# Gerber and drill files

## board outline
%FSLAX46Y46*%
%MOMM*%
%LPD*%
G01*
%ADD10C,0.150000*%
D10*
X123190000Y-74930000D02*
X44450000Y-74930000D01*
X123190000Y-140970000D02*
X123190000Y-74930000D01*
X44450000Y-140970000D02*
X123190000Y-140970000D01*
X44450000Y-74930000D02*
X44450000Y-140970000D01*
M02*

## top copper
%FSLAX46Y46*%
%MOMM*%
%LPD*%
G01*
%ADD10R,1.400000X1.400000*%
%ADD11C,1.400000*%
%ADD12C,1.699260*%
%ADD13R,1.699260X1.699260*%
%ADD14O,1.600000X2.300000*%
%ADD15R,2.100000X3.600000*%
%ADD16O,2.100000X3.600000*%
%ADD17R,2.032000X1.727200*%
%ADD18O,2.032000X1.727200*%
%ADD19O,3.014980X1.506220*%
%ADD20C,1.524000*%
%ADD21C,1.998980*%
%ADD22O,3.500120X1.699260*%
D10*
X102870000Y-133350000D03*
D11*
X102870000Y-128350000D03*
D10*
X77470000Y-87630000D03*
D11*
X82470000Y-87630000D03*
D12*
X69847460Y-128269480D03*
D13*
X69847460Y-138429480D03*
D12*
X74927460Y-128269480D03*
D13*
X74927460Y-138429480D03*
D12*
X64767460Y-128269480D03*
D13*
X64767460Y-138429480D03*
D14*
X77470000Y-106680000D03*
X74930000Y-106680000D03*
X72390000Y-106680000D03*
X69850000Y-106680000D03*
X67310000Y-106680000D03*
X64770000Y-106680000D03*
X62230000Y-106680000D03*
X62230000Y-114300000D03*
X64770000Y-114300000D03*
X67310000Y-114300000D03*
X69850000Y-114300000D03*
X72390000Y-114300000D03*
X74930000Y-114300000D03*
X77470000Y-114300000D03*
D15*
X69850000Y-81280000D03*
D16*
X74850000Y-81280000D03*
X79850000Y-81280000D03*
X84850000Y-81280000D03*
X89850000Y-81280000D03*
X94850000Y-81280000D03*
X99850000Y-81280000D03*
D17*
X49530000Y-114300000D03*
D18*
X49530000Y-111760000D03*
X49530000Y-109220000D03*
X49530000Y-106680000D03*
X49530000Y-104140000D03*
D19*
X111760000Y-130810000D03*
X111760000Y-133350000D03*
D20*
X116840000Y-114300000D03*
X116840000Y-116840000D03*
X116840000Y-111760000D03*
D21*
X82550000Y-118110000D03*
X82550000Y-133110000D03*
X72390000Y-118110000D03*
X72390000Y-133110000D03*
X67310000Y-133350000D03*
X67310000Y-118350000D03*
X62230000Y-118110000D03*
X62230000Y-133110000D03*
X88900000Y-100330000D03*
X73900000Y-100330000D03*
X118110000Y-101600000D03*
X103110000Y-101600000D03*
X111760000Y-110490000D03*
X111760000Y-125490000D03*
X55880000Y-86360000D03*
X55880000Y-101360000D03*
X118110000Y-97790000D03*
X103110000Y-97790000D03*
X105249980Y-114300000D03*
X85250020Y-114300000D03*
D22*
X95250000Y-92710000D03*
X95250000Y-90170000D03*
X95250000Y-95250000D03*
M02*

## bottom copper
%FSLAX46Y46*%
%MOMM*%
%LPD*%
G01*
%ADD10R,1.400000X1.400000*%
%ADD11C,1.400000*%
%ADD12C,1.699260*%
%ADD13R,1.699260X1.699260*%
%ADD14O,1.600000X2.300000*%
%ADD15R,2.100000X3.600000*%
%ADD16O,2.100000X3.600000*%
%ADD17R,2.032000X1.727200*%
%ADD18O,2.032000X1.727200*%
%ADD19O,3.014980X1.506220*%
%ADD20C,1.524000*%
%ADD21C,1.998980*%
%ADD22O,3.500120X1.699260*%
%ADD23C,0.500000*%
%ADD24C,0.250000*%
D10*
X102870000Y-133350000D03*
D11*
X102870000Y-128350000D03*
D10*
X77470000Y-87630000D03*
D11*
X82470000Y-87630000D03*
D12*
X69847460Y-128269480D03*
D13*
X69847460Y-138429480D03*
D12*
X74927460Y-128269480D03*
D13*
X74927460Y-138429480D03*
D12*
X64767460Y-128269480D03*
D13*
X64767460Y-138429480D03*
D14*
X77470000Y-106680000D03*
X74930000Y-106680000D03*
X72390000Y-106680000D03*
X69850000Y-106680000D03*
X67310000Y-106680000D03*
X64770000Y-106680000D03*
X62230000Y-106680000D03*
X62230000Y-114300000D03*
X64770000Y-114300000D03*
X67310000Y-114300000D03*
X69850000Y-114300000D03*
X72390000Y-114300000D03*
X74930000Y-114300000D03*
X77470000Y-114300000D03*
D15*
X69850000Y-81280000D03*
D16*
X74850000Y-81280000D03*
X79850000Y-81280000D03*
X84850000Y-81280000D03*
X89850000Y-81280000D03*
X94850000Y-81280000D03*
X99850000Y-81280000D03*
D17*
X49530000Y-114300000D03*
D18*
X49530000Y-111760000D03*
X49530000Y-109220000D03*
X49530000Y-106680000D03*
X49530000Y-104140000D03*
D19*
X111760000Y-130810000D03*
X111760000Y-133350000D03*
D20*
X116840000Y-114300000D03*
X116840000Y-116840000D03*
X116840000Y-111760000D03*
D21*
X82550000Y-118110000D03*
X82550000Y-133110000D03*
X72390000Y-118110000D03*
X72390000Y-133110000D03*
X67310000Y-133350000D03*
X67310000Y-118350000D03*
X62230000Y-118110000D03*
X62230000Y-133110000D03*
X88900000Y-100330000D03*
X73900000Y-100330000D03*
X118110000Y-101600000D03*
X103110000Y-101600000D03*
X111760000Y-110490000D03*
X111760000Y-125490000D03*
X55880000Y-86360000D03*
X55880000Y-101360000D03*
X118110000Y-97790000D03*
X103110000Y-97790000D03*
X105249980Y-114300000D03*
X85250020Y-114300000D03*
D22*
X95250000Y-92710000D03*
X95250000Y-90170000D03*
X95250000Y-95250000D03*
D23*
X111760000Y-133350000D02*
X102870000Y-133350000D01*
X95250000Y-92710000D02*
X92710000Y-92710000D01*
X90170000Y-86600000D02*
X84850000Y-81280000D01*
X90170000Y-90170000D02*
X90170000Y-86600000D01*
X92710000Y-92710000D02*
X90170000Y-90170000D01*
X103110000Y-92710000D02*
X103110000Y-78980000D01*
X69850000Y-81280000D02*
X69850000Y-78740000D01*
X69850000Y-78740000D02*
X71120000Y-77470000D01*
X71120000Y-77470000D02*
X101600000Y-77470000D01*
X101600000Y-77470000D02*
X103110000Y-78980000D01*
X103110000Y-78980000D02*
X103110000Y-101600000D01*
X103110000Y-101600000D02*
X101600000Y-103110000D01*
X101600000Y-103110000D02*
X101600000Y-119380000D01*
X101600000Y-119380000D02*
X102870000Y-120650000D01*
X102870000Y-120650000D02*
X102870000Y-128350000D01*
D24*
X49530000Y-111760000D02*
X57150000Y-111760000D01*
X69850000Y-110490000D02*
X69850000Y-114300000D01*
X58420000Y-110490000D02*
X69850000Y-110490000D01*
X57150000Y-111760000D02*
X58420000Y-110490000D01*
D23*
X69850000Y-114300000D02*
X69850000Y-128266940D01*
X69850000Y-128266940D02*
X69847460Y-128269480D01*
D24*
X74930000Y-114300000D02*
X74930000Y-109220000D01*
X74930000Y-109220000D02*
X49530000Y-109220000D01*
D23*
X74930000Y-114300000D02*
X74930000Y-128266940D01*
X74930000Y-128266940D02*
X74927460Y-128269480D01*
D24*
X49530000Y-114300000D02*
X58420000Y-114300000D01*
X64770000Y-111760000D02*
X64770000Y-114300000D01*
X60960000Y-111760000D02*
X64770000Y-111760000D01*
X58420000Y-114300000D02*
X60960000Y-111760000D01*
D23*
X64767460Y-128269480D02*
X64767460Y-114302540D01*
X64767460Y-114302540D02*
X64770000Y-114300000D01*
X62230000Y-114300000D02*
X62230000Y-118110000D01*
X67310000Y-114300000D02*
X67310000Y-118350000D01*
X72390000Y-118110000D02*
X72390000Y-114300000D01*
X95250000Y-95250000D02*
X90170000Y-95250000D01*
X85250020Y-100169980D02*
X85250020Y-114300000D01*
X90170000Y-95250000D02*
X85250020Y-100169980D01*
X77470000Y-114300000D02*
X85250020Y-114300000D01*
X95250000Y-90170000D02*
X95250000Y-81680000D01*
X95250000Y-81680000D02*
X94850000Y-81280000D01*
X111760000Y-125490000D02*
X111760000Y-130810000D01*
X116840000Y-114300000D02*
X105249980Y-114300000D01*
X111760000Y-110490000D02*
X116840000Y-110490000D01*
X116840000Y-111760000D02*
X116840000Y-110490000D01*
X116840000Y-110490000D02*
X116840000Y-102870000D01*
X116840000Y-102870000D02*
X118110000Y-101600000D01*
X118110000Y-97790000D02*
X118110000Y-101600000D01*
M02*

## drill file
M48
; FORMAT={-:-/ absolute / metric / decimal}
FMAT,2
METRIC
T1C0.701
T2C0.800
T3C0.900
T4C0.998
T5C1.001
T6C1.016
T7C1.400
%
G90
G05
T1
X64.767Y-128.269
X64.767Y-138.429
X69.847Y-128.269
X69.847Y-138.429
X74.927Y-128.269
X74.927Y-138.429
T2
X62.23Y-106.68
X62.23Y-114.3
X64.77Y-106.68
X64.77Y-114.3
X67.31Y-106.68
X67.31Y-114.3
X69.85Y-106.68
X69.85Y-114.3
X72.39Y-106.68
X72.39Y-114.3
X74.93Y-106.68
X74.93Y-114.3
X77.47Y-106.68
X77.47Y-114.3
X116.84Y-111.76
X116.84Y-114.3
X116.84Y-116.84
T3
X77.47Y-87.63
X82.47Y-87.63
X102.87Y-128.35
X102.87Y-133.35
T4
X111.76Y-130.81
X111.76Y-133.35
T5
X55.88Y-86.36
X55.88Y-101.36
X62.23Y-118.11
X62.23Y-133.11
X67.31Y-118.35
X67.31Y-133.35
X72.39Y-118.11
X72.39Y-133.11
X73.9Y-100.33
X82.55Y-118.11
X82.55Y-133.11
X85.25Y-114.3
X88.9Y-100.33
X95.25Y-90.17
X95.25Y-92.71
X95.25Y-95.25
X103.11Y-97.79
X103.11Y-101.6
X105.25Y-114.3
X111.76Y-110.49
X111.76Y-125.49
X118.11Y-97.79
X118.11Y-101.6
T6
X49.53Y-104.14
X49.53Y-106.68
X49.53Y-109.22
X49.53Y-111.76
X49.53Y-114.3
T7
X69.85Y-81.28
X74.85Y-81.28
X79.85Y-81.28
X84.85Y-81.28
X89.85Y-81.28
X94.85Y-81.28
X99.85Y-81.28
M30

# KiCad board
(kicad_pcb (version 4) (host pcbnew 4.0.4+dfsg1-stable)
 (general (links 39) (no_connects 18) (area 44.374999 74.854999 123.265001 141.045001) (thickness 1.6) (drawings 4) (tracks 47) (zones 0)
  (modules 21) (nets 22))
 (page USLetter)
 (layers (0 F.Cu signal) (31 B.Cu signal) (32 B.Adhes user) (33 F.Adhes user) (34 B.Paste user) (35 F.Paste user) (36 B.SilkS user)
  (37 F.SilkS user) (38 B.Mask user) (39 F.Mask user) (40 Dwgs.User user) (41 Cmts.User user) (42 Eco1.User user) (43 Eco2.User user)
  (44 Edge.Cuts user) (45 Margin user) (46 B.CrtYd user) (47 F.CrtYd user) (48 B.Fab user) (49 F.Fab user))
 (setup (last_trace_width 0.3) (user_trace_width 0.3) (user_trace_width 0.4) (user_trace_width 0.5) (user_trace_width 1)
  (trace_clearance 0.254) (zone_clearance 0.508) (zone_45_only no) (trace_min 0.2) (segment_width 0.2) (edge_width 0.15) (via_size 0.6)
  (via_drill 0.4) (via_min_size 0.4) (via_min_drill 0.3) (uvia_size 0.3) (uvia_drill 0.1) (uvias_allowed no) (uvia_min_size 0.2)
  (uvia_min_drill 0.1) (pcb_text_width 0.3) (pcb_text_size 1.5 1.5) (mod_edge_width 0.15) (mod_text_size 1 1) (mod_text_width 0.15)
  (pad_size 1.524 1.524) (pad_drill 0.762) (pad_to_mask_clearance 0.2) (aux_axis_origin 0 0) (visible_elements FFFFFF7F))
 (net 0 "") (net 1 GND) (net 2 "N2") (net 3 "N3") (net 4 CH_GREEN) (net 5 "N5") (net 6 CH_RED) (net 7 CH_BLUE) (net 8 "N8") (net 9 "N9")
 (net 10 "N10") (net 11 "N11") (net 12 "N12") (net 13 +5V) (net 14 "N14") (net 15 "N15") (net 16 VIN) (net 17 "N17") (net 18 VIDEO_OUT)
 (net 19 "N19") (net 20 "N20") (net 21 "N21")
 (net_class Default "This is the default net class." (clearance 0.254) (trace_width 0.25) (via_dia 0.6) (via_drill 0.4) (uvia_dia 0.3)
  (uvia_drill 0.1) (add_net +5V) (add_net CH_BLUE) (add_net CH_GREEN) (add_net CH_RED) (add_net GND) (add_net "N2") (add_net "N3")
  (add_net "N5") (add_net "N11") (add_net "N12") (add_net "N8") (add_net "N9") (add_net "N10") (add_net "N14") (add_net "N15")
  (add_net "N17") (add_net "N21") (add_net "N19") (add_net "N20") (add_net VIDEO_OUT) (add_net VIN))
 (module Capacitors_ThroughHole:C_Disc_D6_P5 (layer F.Cu) (at 102.87 133.35 90)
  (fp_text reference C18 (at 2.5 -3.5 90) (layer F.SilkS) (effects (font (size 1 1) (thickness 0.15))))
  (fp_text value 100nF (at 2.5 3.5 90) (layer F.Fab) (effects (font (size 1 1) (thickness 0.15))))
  (pad 1 thru_hole rect (at 0 0 90) (size 1.4 1.4) (drill 0.9) (layers *.Cu *.Mask F.SilkS) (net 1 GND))
  (pad 2 thru_hole circle (at 5 0 90) (size 1.4 1.4) (drill 0.9) (layers *.Cu *.Mask F.SilkS) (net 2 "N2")))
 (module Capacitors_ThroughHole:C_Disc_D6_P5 (layer F.Cu) (at 77.47 87.63)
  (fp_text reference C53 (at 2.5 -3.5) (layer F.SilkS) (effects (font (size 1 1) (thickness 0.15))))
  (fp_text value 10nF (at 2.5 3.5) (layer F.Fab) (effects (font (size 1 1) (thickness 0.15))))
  (pad 1 thru_hole rect (at 0 0) (size 1.4 1.4) (drill 0.9) (layers *.Cu *.Mask F.SilkS) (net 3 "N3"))
  (pad 2 thru_hole circle (at 5 0) (size 1.4 1.4) (drill 0.9) (layers *.Cu *.Mask F.SilkS) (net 1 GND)))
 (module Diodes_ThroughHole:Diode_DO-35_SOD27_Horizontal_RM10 (layer F.Cu) (at 69.85 138.43 90)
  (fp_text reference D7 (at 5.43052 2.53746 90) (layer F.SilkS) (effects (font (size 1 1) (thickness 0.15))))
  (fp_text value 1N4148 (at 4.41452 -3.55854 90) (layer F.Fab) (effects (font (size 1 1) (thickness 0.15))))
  (pad 2 thru_hole circle (at 10.16052 -0.00254 270) (size 1.69926 1.69926) (drill 0.70104) (layers *.Cu *.Mask F.SilkS) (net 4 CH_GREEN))
  (pad 1 thru_hole rect (at 0.00052 -0.00254 270) (size 1.69926 1.69926) (drill 0.70104) (layers *.Cu *.Mask F.SilkS) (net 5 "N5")))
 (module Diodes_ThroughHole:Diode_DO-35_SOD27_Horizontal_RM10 (layer F.Cu) (at 74.93 138.43 90)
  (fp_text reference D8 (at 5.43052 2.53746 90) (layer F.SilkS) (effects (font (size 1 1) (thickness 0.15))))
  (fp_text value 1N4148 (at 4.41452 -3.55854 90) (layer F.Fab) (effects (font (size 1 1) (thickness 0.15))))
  (pad 2 thru_hole circle (at 10.16052 -0.00254 270) (size 1.69926 1.69926) (drill 0.70104) (layers *.Cu *.Mask F.SilkS) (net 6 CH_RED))
  (pad 1 thru_hole rect (at 0.00052 -0.00254 270) (size 1.69926 1.69926) (drill 0.70104) (layers *.Cu *.Mask F.SilkS) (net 5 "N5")))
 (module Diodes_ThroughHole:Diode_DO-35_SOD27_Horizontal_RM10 (layer F.Cu) (at 64.77 138.43 90)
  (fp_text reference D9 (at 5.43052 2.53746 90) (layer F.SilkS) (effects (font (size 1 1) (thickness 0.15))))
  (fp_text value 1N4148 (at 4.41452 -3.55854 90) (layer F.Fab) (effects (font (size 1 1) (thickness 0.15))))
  (pad 2 thru_hole circle (at 10.16052 -0.00254 270) (size 1.69926 1.69926) (drill 0.70104) (layers *.Cu *.Mask F.SilkS) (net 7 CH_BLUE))
  (pad 1 thru_hole rect (at 0.00052 -0.00254 270) (size 1.69926 1.69926) (drill 0.70104) (layers *.Cu *.Mask F.SilkS) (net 5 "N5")))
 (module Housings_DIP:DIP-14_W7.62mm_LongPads (layer F.Cu) (at 77.47 106.68 270)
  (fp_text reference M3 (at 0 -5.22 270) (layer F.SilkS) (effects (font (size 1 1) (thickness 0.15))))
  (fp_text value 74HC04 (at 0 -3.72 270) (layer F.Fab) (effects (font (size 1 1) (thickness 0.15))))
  (pad 1 thru_hole oval (at 0 0 270) (size 2.3 1.6) (drill 0.8) (layers *.Cu *.Mask F.SilkS))
  (pad 2 thru_hole oval (at 0 2.54 270) (size 2.3 1.6) (drill 0.8) (layers *.Cu *.Mask F.SilkS))
  (pad 3 thru_hole oval (at 0 5.08 270) (size 2.3 1.6) (drill 0.8) (layers *.Cu *.Mask F.SilkS))
  (pad 4 thru_hole oval (at 0 7.62 270) (size 2.3 1.6) (drill 0.8) (layers *.Cu *.Mask F.SilkS))
  (pad 5 thru_hole oval (at 0 10.16 270) (size 2.3 1.6) (drill 0.8) (layers *.Cu *.Mask F.SilkS) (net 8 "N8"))
  (pad 6 thru_hole oval (at 0 12.7 270) (size 2.3 1.6) (drill 0.8) (layers *.Cu *.Mask F.SilkS) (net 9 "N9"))
  (pad 7 thru_hole oval (at 0 15.24 270) (size 2.3 1.6) (drill 0.8) (layers *.Cu *.Mask F.SilkS) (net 1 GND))
  (pad 8 thru_hole oval (at 7.62 15.24 270) (size 2.3 1.6) (drill 0.8) (layers *.Cu *.Mask F.SilkS) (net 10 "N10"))
  (pad 9 thru_hole oval (at 7.62 12.7 270) (size 2.3 1.6) (drill 0.8) (layers *.Cu *.Mask F.SilkS) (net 7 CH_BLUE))
  (pad 10 thru_hole oval (at 7.62 10.16 270) (size 2.3 1.6) (drill 0.8) (layers *.Cu *.Mask F.SilkS) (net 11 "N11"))
  (pad 11 thru_hole oval (at 7.62 7.62 270) (size 2.3 1.6) (drill 0.8) (layers *.Cu *.Mask F.SilkS) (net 4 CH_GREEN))
  (pad 12 thru_hole oval (at 7.62 5.08 270) (size 2.3 1.6) (drill 0.8) (layers *.Cu *.Mask F.SilkS) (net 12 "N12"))
  (pad 13 thru_hole oval (at 7.62 2.54 270) (size 2.3 1.6) (drill 0.8) (layers *.Cu *.Mask F.SilkS) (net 6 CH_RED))
  (pad 14 thru_hole oval (at 7.62 0 270) (size 2.3 1.6) (drill 0.8) (layers *.Cu *.Mask F.SilkS) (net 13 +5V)))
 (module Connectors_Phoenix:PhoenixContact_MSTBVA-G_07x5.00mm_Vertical (layer F.Cu) (at 69.85 81.28)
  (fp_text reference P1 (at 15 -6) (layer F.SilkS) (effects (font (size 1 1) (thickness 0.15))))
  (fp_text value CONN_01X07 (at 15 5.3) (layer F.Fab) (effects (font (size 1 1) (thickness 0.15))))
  (pad 1 thru_hole rect (at 0 0) (size 2.1 3.6) (drill 1.4) (layers *.Cu *.Mask) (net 2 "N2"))
  (pad 2 thru_hole oval (at 5 0) (size 2.1 3.6) (drill 1.4) (layers *.Cu *.Mask) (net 3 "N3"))
  (pad 3 thru_hole oval (at 10 0) (size 2.1 3.6) (drill 1.4) (layers *.Cu *.Mask) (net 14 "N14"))
  (pad 4 thru_hole oval (at 15 0) (size 2.1 3.6) (drill 1.4) (layers *.Cu *.Mask) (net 1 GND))
  (pad 5 thru_hole oval (at 20 0) (size 2.1 3.6) (drill 1.4) (layers *.Cu *.Mask) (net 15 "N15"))
  (pad 6 thru_hole oval (at 25 0) (size 2.1 3.6) (drill 1.4) (layers *.Cu *.Mask) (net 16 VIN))
  (pad 7 thru_hole oval (at 30 0) (size 2.1 3.6) (drill 1.4) (layers *.Cu *.Mask) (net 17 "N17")))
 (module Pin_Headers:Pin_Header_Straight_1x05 (layer B.Cu) (at 49.53 114.3)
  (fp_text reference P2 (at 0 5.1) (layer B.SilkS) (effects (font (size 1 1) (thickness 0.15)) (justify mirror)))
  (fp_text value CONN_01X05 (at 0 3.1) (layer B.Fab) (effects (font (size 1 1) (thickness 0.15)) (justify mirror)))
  (pad 1 thru_hole rect (at 0 0) (size 2.032 1.7272) (drill 1.016) (layers *.Cu *.Mask B.SilkS) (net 7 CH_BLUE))
  (pad 2 thru_hole oval (at 0 -2.54) (size 2.032 1.7272) (drill 1.016) (layers *.Cu *.Mask B.SilkS) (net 4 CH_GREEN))
  (pad 3 thru_hole oval (at 0 -5.08) (size 2.032 1.7272) (drill 1.016) (layers *.Cu *.Mask B.SilkS) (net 6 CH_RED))
  (pad 4 thru_hole oval (at 0 -7.62) (size 2.032 1.7272) (drill 1.016) (layers *.Cu *.Mask B.SilkS) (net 13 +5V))
  (pad 5 thru_hole oval (at 0 -10.16) (size 2.032 1.7272) (drill 1.016) (layers *.Cu *.Mask B.SilkS) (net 1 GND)))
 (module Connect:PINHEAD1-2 (layer F.Cu) (at 111.76 132.08 270)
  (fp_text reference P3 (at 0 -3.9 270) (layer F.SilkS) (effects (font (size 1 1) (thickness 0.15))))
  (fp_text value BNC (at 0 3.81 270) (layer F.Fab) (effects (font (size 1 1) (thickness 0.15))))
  (pad 1 thru_hole oval (at -1.27 0 270) (size 1.50622 3.01498) (drill 0.99822) (layers *.Cu *.Mask) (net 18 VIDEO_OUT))
  (pad 2 thru_hole oval (at 1.27 0 270) (size 1.50622 3.01498) (drill 0.99822) (layers *.Cu *.Mask) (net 1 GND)))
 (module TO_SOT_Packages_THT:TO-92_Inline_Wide (layer F.Cu) (at 116.84 111.76 270)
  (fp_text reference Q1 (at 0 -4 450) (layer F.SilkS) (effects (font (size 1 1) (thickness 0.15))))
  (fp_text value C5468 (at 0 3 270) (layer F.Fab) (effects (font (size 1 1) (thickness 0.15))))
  (pad 2 thru_hole circle (at 2.54 0) (size 1.524 1.524) (drill 0.8) (layers *.Cu *.Mask F.SilkS) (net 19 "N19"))
  (pad 3 thru_hole circle (at 5.08 0) (size 1.524 1.524) (drill 0.8) (layers *.Cu *.Mask F.SilkS) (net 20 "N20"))
  (pad 1 thru_hole circle (at 0 0) (size 1.524 1.524) (drill 0.8) (layers *.Cu *.Mask F.SilkS) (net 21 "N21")))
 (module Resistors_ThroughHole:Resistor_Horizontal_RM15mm (layer F.Cu) (at 82.55 118.11 270)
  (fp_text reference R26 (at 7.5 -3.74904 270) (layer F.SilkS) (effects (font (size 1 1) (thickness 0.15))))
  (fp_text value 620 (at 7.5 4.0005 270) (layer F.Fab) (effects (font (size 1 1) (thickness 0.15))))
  (pad 1 thru_hole circle (at 0 0 270) (size 1.99898 1.99898) (drill 1.00076) (layers *.Cu *.SilkS *.Mask) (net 9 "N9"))
  (pad 2 thru_hole circle (at 15 0 270) (size 1.99898 1.99898) (drill 1.00076) (layers *.Cu *.SilkS *.Mask) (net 20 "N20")))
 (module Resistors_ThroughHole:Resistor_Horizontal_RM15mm (layer F.Cu) (at 72.39 118.11 270)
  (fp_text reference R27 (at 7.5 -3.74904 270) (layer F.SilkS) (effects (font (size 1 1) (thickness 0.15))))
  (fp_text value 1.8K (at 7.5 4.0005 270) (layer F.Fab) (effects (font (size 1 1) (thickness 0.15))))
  (pad 1 thru_hole circle (at 0 0 270) (size 1.99898 1.99898) (drill 1.00076) (layers *.Cu *.SilkS *.Mask) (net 12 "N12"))
  (pad 2 thru_hole circle (at 15 0 270) (size 1.99898 1.99898) (drill 1.00076) (layers *.Cu *.SilkS *.Mask) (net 20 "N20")))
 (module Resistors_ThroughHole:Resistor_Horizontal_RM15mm (layer F.Cu) (at 67.31 133.35 90)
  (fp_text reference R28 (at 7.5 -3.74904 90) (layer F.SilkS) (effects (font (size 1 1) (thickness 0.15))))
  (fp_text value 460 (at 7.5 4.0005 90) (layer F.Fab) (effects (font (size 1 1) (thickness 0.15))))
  (pad 1 thru_hole circle (at 0 0 90) (size 1.99898 1.99898) (drill 1.00076) (layers *.Cu *.SilkS *.Mask) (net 20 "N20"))
  (pad 2 thru_hole circle (at 15 0 90) (size 1.99898 1.99898) (drill 1.00076) (layers *.Cu *.SilkS *.Mask) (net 11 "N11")))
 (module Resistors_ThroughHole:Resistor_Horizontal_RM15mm (layer F.Cu) (at 62.23 118.11 270)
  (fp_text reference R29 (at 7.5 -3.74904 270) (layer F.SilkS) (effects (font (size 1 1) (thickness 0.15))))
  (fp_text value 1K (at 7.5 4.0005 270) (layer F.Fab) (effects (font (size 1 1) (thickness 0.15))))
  (pad 1 thru_hole circle (at 0 0 270) (size 1.99898 1.99898) (drill 1.00076) (layers *.Cu *.SilkS *.Mask) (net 10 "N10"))
  (pad 2 thru_hole circle (at 15 0 270) (size 1.99898 1.99898) (drill 1.00076) (layers *.Cu *.SilkS *.Mask) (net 20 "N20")))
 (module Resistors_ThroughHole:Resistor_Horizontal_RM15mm (layer F.Cu) (at 88.9 100.33 180)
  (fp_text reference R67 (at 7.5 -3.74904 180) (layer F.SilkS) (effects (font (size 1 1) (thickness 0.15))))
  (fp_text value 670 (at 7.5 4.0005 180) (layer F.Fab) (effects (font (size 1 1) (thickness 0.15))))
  (pad 1 thru_hole circle (at 0 0 180) (size 1.99898 1.99898) (drill 1.00076) (layers *.Cu *.SilkS *.Mask) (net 5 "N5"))
  (pad 2 thru_hole circle (at 15 0 180) (size 1.99898 1.99898) (drill 1.00076) (layers *.Cu *.SilkS *.Mask) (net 8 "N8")))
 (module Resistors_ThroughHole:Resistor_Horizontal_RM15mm (layer F.Cu) (at 118.11 101.6 180)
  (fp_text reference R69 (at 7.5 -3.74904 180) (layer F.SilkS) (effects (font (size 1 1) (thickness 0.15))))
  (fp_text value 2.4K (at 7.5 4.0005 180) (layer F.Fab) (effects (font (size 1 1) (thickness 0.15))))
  (pad 1 thru_hole circle (at 0 0 180) (size 1.99898 1.99898) (drill 1.00076) (layers *.Cu *.SilkS *.Mask) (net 21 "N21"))
  (pad 2 thru_hole circle (at 15 0 180) (size 1.99898 1.99898) (drill 1.00076) (layers *.Cu *.SilkS *.Mask) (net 2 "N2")))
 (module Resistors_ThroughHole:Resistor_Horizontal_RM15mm (layer F.Cu) (at 111.76 110.49 270)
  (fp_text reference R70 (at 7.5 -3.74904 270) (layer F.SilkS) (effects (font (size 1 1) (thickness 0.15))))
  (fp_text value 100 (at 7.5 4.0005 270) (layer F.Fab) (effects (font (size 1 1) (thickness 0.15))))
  (pad 1 thru_hole circle (at 0 0 270) (size 1.99898 1.99898) (drill 1.00076) (layers *.Cu *.SilkS *.Mask) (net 21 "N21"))
  (pad 2 thru_hole circle (at 15 0 270) (size 1.99898 1.99898) (drill 1.00076) (layers *.Cu *.SilkS *.Mask) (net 18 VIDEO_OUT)))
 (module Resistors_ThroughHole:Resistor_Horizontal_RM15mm (layer F.Cu) (at 55.88 86.36 270)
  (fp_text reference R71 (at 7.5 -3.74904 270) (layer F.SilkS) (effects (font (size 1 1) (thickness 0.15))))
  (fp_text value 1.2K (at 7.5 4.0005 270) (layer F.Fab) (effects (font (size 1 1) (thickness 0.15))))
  (pad 1 thru_hole circle (at 0 0 270) (size 1.99898 1.99898) (drill 1.00076) (layers *.Cu *.SilkS *.Mask) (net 3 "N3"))
  (pad 2 thru_hole circle (at 15 0 270) (size 1.99898 1.99898) (drill 1.00076) (layers *.Cu *.SilkS *.Mask) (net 20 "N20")))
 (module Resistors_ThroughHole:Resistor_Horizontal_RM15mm (layer F.Cu) (at 118.11 97.79 180)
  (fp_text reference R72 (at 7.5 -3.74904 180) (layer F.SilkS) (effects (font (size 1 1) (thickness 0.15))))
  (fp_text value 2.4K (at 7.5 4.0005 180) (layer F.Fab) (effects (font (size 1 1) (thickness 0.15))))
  (pad 1 thru_hole circle (at 0 0 180) (size 1.99898 1.99898) (drill 1.00076) (layers *.Cu *.SilkS *.Mask) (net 21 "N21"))
  (pad 2 thru_hole circle (at 15 0 180) (size 1.99898 1.99898) (drill 1.00076) (layers *.Cu *.SilkS *.Mask) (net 2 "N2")))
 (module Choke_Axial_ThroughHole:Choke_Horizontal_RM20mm (layer F.Cu) (at 95.25 114.3 180)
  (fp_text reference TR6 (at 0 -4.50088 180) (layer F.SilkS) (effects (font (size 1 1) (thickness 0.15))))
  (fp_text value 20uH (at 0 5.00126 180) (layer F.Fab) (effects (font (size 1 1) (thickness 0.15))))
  (pad 1 thru_hole circle (at -9.99998 0 180) (size 1.99898 1.99898) (drill 1.00076) (layers *.Cu *.Mask F.SilkS) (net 19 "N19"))
  (pad 2 thru_hole circle (at 9.99998 0 180) (size 1.99898 1.99898) (drill 1.00076) (layers *.Cu *.Mask F.SilkS) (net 13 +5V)))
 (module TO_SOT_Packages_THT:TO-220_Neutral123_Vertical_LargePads (layer F.Cu) (at 95.25 92.71 270)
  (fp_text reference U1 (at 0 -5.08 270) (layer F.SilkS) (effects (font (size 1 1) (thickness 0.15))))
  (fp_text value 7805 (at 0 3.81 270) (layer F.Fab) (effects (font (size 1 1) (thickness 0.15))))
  (pad 2 thru_hole oval (at 0 0) (size 3.50012 1.69926) (drill 1.00076) (layers *.Cu *.Mask F.SilkS) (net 1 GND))
  (pad 1 thru_hole oval (at -2.54 0) (size 3.50012 1.69926) (drill 1.00076) (layers *.Cu *.Mask F.SilkS) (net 16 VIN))
  (pad 3 thru_hole oval (at 2.54 0) (size 3.50012 1.69926) (drill 1.00076) (layers *.Cu *.Mask F.SilkS) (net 13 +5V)))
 (gr_line (start 123.19 74.93) (end 44.45 74.93) (angle 90) (layer Edge.Cuts) (width 0.15))
 (gr_line (start 123.19 140.97) (end 123.19 74.93) (angle 90) (layer Edge.Cuts) (width 0.15))
 (gr_line (start 44.45 140.97) (end 123.19 140.97) (angle 90) (layer Edge.Cuts) (width 0.15))
 (gr_line (start 44.45 74.93) (end 44.45 140.97) (angle 90) (layer Edge.Cuts) (width 0.15))
 (segment (start 111.76 133.35) (end 102.87 133.35) (width 0.5) (layer B.Cu) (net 1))
 (segment (start 95.25 92.71) (end 92.71 92.71) (width 0.5) (layer B.Cu) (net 1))
 (segment (start 90.17 86.6) (end 84.85 81.28) (width 0.5) (layer B.Cu) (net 1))
 (segment (start 90.17 90.17) (end 90.17 86.6) (width 0.5) (layer B.Cu) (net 1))
 (segment (start 92.71 92.71) (end 90.17 90.17) (width 0.5) (layer B.Cu) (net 1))
 (segment (start 103.11 92.71) (end 103.11 78.98) (width 0.5) (layer B.Cu) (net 2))
 (segment (start 69.85 81.28) (end 69.85 78.74) (width 0.5) (layer B.Cu) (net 2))
 (segment (start 69.85 78.74) (end 71.12 77.47) (width 0.5) (layer B.Cu) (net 2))
 (segment (start 71.12 77.47) (end 101.6 77.47) (width 0.5) (layer B.Cu) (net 2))
 (segment (start 101.6 77.47) (end 103.11 78.98) (width 0.5) (layer B.Cu) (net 2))
 (segment (start 103.11 78.98) (end 103.11 101.6) (width 0.5) (layer B.Cu) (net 2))
 (segment (start 103.11 101.6) (end 101.6 103.11) (width 0.5) (layer B.Cu) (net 2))
 (segment (start 101.6 103.11) (end 101.6 119.38) (width 0.5) (layer B.Cu) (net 2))
 (segment (start 101.6 119.38) (end 102.87 120.65) (width 0.5) (layer B.Cu) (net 2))
 (segment (start 102.87 120.65) (end 102.87 128.35) (width 0.5) (layer B.Cu) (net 2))
 (segment (start 49.53 111.76) (end 57.15 111.76) (width 0.25) (layer B.Cu) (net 4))
 (segment (start 69.85 110.49) (end 69.85 114.3) (width 0.25) (layer B.Cu) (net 4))
 (segment (start 58.42 110.49) (end 69.85 110.49) (width 0.25) (layer B.Cu) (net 4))
 (segment (start 57.15 111.76) (end 58.42 110.49) (width 0.25) (layer B.Cu) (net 4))
 (segment (start 69.85 114.3) (end 69.85 128.26694) (width 0.5) (layer B.Cu) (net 4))
 (segment (start 69.85 128.26694) (end 69.84746 128.26948) (width 0.5) (layer B.Cu) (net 4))
 (segment (start 74.93 114.3) (end 74.93 109.22) (width 0.25) (layer B.Cu) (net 6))
 (segment (start 74.93 109.22) (end 49.53 109.22) (width 0.25) (layer B.Cu) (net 6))
 (segment (start 74.93 114.3) (end 74.93 128.26694) (width 0.5) (layer B.Cu) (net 6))
 (segment (start 74.93 128.26694) (end 74.92746 128.26948) (width 0.5) (layer B.Cu) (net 6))
 (segment (start 49.53 114.3) (end 58.42 114.3) (width 0.25) (layer B.Cu) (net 7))
 (segment (start 64.77 111.76) (end 64.77 114.3) (width 0.25) (layer B.Cu) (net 7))
 (segment (start 60.96 111.76) (end 64.77 111.76) (width 0.25) (layer B.Cu) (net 7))
 (segment (start 58.42 114.3) (end 60.96 111.76) (width 0.25) (layer B.Cu) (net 7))
 (segment (start 64.76746 128.26948) (end 64.76746 114.30254) (width 0.5) (layer B.Cu) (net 7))
 (segment (start 64.76746 114.30254) (end 64.77 114.3) (width 0.5) (layer B.Cu) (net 7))
 (segment (start 62.23 114.3) (end 62.23 118.11) (width 0.5) (layer B.Cu) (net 10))
 (segment (start 67.31 114.3) (end 67.31 118.35) (width 0.5) (layer B.Cu) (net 11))
 (segment (start 72.39 118.11) (end 72.39 114.3) (width 0.5) (layer B.Cu) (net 12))
 (segment (start 95.25 95.25) (end 90.17 95.25) (width 0.5) (layer B.Cu) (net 13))
 (segment (start 85.25002 100.16998) (end 85.25002 114.3) (width 0.5) (layer B.Cu) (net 13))
 (segment (start 90.17 95.25) (end 85.25002 100.16998) (width 0.5) (layer B.Cu) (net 13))
 (segment (start 77.47 114.3) (end 85.25002 114.3) (width 0.5) (layer B.Cu) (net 13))
 (segment (start 95.25 90.17) (end 95.25 81.68) (width 0.5) (layer B.Cu) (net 16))
 (segment (start 95.25 81.68) (end 94.85 81.28) (width 0.5) (layer B.Cu) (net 16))
 (segment (start 111.76 125.49) (end 111.76 130.81) (width 0.5) (layer B.Cu) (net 18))
 (segment (start 116.84 114.3) (end 105.24998 114.3) (width 0.5) (layer B.Cu) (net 19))
 (segment (start 111.76 110.49) (end 116.84 110.49) (width 0.5) (layer B.Cu) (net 21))
 (segment (start 116.84 111.76) (end 116.84 110.49) (width 0.5) (layer B.Cu) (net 21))
 (segment (start 116.84 110.49) (end 116.84 102.87) (width 0.5) (layer B.Cu) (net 21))
 (segment (start 116.84 102.87) (end 118.11 101.6) (width 0.5) (layer B.Cu) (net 21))
 (segment (start 118.11 97.79) (end 118.11 101.6) (width 0.5) (layer B.Cu) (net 21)))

